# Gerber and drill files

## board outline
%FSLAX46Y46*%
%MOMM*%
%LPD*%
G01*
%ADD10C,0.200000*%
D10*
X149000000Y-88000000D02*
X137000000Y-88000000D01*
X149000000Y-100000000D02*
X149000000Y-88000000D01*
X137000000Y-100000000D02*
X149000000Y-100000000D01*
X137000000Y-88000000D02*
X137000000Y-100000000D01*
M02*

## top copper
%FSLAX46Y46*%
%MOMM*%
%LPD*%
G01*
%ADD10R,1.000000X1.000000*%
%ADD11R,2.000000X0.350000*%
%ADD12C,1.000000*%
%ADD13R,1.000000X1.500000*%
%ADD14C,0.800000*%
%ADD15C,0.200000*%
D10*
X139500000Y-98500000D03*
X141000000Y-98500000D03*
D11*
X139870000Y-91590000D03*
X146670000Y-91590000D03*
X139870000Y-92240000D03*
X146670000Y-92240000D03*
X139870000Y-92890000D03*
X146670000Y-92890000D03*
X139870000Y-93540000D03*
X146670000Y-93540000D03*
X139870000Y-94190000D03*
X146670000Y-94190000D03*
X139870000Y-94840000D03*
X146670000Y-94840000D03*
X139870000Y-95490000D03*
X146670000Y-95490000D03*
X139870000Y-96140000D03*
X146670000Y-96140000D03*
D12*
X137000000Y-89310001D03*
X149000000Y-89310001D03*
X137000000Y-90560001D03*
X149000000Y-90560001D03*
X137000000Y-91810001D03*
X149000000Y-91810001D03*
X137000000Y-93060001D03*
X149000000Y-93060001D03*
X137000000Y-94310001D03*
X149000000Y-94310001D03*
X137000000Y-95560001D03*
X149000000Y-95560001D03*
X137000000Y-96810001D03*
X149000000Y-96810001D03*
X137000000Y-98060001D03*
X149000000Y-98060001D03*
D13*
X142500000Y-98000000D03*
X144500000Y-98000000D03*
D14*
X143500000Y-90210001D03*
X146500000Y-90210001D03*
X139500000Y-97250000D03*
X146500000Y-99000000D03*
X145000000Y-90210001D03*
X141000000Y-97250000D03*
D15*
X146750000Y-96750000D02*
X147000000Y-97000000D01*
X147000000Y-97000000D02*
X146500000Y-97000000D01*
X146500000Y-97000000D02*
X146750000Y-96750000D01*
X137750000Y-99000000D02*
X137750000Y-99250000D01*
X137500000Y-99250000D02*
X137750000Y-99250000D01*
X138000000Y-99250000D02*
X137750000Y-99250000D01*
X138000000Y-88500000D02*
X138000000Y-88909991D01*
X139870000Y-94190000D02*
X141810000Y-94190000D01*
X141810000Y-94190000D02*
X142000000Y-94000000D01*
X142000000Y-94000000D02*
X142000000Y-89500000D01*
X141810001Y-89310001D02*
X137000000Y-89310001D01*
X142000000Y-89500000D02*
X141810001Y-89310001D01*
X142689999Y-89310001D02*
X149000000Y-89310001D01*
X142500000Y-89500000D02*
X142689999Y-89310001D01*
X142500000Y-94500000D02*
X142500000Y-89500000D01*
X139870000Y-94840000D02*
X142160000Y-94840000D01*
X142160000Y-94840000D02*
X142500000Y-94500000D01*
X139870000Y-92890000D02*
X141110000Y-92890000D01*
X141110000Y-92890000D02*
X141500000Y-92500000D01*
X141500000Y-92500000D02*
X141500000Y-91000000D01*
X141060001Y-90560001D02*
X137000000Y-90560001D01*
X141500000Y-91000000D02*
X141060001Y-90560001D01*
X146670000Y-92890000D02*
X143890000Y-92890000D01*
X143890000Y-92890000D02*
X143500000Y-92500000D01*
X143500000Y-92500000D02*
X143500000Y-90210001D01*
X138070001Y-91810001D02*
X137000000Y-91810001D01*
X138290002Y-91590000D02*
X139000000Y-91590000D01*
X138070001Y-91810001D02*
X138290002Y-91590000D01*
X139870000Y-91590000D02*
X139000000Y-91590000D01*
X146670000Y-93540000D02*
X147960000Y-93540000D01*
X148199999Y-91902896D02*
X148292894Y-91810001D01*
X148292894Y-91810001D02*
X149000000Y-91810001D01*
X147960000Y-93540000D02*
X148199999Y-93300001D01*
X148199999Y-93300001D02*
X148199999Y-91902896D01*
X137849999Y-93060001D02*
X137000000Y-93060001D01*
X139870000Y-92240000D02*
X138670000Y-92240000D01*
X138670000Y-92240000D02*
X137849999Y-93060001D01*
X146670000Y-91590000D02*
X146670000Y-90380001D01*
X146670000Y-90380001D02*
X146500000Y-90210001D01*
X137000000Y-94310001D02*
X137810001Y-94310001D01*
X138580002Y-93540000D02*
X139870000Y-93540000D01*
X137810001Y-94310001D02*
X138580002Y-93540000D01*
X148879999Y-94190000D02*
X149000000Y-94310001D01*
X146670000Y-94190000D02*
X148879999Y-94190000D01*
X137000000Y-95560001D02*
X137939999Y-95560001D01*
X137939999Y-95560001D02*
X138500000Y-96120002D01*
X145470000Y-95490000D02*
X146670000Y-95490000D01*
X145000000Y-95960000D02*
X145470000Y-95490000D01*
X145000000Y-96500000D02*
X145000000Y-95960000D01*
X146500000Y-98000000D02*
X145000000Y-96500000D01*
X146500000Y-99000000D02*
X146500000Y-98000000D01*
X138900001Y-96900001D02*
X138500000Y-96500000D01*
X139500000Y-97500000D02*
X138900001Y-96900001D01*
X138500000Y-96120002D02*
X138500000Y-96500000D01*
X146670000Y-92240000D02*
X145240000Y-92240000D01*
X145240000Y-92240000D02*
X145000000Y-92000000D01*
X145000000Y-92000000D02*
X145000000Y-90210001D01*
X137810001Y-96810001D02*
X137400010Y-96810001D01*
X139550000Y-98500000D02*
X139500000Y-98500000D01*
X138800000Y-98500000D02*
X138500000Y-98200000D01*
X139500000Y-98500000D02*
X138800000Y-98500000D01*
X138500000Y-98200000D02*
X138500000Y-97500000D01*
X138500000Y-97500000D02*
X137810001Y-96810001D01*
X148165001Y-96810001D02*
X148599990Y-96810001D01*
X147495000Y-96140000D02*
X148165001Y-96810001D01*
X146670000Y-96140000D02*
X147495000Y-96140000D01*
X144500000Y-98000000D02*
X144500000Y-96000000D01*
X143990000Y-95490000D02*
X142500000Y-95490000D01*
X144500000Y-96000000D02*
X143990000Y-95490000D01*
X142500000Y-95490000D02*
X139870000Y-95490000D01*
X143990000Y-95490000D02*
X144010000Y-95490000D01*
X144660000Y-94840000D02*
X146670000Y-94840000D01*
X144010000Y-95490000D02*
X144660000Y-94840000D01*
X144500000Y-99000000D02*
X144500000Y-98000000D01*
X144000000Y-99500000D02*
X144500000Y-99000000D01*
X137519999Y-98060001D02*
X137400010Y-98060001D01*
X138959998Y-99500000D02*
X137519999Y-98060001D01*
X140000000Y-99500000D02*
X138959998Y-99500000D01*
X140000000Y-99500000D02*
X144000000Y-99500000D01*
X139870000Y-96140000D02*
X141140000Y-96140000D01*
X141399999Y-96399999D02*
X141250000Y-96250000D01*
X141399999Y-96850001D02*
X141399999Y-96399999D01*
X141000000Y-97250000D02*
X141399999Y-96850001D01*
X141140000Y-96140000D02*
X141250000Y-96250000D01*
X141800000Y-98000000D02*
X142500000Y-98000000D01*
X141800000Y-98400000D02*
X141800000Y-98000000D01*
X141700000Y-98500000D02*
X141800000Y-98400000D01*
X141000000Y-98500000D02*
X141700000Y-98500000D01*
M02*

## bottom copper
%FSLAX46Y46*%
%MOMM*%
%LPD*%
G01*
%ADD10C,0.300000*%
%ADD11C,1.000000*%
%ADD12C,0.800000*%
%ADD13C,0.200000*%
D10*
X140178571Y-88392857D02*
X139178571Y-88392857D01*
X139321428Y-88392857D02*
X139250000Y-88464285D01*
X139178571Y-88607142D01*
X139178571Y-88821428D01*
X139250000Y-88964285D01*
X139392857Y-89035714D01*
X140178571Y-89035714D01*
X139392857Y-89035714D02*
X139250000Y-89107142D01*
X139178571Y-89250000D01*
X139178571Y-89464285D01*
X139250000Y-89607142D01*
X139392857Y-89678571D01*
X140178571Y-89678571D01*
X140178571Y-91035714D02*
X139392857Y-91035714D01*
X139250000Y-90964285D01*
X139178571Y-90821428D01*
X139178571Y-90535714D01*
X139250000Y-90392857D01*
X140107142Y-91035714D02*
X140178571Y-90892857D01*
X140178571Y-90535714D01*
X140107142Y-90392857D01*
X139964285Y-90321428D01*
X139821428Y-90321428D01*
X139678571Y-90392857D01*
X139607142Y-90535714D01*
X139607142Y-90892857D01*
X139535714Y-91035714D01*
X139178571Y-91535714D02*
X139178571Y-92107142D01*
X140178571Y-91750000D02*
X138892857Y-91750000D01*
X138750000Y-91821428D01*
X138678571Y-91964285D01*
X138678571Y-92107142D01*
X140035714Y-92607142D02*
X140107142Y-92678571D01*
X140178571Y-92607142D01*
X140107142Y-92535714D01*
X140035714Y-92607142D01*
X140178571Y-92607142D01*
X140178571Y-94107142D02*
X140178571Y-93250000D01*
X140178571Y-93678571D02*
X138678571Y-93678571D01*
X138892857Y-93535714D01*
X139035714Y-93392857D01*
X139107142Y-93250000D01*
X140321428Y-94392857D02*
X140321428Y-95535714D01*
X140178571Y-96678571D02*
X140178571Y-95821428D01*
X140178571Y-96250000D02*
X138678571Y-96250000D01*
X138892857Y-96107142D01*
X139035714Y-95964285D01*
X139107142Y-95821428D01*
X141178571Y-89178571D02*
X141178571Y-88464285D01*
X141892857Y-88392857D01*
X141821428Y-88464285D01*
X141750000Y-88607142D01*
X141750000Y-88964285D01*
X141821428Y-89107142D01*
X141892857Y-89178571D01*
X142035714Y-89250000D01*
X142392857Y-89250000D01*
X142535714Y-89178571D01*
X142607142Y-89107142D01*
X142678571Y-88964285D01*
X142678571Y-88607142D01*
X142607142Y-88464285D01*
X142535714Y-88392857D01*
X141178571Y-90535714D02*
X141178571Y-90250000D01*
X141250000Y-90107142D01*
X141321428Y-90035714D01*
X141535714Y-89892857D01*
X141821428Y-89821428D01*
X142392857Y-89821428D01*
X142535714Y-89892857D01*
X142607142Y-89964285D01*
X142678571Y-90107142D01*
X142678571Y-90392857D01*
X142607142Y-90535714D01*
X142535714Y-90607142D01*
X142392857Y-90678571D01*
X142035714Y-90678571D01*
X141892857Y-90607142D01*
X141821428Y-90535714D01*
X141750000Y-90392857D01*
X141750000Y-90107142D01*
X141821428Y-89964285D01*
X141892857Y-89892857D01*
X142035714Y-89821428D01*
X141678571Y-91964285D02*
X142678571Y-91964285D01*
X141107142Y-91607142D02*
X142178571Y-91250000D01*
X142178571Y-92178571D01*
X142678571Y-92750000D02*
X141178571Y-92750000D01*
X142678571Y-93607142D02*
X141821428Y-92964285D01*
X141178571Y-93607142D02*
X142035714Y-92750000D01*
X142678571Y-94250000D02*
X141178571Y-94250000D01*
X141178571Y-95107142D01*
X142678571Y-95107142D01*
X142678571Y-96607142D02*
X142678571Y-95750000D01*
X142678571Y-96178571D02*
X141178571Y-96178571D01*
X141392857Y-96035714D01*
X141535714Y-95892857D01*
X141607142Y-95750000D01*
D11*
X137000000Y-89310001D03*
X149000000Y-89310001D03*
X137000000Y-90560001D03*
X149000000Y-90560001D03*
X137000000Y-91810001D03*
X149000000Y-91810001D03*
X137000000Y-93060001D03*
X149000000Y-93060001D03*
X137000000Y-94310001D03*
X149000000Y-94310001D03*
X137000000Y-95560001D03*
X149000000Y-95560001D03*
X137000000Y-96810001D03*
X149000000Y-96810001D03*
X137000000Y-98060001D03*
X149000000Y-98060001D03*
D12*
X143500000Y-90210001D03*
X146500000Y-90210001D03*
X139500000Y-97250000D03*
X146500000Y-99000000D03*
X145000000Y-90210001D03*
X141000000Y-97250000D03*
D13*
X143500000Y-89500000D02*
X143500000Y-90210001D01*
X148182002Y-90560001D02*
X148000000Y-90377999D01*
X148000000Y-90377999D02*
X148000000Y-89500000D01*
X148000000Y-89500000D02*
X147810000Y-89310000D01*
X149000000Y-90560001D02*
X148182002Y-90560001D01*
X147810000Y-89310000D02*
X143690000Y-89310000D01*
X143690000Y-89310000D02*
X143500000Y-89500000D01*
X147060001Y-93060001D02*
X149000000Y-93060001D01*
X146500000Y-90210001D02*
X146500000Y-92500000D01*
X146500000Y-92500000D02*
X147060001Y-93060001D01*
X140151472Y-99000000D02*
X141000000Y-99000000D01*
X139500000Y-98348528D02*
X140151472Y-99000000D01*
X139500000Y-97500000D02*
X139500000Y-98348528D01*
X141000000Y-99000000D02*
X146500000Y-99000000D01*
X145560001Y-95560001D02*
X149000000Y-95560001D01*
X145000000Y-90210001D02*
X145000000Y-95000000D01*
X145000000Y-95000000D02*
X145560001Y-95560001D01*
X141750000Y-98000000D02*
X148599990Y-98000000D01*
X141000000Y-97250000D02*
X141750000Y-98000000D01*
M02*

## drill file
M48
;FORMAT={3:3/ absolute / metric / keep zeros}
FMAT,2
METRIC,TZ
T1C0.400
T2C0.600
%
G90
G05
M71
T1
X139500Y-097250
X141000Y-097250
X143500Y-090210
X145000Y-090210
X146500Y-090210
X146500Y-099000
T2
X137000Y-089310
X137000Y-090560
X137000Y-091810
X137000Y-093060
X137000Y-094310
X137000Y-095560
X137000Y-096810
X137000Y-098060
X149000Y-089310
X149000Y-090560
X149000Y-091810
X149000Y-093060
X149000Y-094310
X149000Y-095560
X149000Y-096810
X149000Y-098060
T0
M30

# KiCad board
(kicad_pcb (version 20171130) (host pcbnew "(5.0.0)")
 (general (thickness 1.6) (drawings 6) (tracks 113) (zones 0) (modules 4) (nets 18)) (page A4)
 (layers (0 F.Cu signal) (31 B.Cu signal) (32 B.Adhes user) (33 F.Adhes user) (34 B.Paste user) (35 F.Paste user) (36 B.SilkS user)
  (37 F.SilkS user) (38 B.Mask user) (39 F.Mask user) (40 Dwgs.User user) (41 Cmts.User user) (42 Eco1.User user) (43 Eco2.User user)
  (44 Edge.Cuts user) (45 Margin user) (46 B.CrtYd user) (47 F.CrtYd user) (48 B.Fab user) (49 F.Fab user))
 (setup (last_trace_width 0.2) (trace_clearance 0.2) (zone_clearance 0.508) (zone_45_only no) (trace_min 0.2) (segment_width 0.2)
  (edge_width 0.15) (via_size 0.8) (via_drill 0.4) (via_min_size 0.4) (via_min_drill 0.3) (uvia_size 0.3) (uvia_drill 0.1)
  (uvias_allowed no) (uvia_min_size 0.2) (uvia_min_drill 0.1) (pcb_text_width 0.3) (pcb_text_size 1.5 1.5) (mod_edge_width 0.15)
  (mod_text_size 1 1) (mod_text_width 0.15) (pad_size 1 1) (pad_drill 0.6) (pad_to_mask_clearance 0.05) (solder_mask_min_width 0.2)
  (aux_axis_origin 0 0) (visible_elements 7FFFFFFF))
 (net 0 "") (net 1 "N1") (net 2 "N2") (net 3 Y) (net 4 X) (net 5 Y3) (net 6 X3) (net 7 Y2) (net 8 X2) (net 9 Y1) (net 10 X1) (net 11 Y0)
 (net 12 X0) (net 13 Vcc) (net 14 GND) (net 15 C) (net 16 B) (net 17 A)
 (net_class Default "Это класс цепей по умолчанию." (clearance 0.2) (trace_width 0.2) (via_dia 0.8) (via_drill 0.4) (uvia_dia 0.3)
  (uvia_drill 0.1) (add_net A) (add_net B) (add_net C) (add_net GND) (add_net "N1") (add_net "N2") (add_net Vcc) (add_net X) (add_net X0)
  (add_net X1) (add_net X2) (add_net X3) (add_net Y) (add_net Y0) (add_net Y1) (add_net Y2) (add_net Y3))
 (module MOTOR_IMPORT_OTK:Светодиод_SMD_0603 (layer F.Cu) (at 141 98.5 180)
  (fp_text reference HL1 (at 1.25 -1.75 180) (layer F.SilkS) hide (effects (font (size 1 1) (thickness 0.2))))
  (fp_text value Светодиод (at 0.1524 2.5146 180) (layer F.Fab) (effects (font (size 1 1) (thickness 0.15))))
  (pad 2 smd rect (at 1.5 0 180) (size 1 1) (layers F.Cu F.Paste F.Mask) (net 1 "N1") (clearance 0.2))
  (pad 1 smd rect (at 0 0 180) (size 1 1) (layers F.Cu F.Paste F.Mask) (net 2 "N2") (clearance 0.2)))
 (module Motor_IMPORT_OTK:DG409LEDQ (layer F.Cu) (at 145.5 89.5 180)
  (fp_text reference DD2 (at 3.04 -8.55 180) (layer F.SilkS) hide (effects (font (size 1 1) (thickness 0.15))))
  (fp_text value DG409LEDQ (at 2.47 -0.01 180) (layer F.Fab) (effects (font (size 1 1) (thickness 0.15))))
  (pad 9 smd rect (at 5.63 -2.09 180) (size 2 0.35) (layers F.Cu F.Paste F.Mask) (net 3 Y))
  (pad 8 smd rect (at -1.17 -2.09 180) (size 2 0.35) (layers F.Cu F.Paste F.Mask) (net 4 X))
  (pad 10 smd rect (at 5.63 -2.74 180) (size 2 0.35) (layers F.Cu F.Paste F.Mask) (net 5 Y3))
  (pad 7 smd rect (at -1.17 -2.74 180) (size 2 0.35) (layers F.Cu F.Paste F.Mask) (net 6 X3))
  (pad 11 smd rect (at 5.63 -3.39 180) (size 2 0.35) (layers F.Cu F.Paste F.Mask) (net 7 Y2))
  (pad 6 smd rect (at -1.17 -3.39 180) (size 2 0.35) (layers F.Cu F.Paste F.Mask) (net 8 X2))
  (pad 12 smd rect (at 5.63 -4.04 180) (size 2 0.35) (layers F.Cu F.Paste F.Mask) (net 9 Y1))
  (pad 5 smd rect (at -1.17 -4.04 180) (size 2 0.35) (layers F.Cu F.Paste F.Mask) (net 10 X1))
  (pad 13 smd rect (at 5.63 -4.69 180) (size 2 0.35) (layers F.Cu F.Paste F.Mask) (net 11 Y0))
  (pad 4 smd rect (at -1.17 -4.69 180) (size 2 0.35) (layers F.Cu F.Paste F.Mask) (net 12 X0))
  (pad 14 smd rect (at 5.63 -5.34 180) (size 2 0.35) (layers F.Cu F.Paste F.Mask) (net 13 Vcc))
  (pad 3 smd rect (at -1.17 -5.34 180) (size 2 0.35) (layers F.Cu F.Paste F.Mask) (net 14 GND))
  (pad 15 smd rect (at 5.63 -5.99 180) (size 2 0.35) (layers F.Cu F.Paste F.Mask) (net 14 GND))
  (pad 2 smd rect (at -1.17 -5.99 180) (size 2 0.35) (layers F.Cu F.Paste F.Mask) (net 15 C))
  (pad 16 smd rect (at 5.63 -6.64 180) (size 2 0.35) (layers F.Cu F.Paste F.Mask) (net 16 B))
  (pad 1 smd rect (at -1.17 -6.64 180) (size 2 0.35) (layers F.Cu F.Paste F.Mask) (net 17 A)))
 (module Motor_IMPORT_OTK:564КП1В (layer F.Cu) (at 137 106.650001)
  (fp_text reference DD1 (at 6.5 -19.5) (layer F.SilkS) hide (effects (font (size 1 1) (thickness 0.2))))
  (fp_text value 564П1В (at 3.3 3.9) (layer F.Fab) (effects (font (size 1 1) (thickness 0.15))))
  (pad 1 thru_hole circle (at 0 -17.34) (size 1 1) (drill 0.6) (layers *.Cu *.Mask) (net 11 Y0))
  (pad 16 thru_hole circle (at 12 -17.34) (size 1 1) (drill 0.6) (layers *.Cu *.Mask) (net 13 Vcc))
  (pad 2 thru_hole circle (at 0 -16.09) (size 1 1) (drill 0.6) (layers *.Cu *.Mask) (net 7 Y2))
  (pad 15 thru_hole circle (at 12 -16.09) (size 1 1) (drill 0.6) (layers *.Cu *.Mask) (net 8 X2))
  (pad 3 thru_hole circle (at 0 -14.84) (size 1 1) (drill 0.6) (layers *.Cu *.Mask) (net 3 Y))
  (pad 14 thru_hole circle (at 12 -14.84) (size 1 1) (drill 0.6) (layers *.Cu *.Mask) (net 10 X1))
  (pad 4 thru_hole circle (at 0 -13.59) (size 1 1) (drill 0.6) (layers *.Cu *.Mask) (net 5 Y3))
  (pad 13 thru_hole circle (at 12 -13.59) (size 1 1) (drill 0.6) (layers *.Cu *.Mask) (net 4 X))
  (pad 5 thru_hole circle (at 0 -12.34) (size 1 1) (drill 0.6) (layers *.Cu *.Mask) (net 9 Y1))
  (pad 12 thru_hole circle (at 12 -12.34) (size 1 1) (drill 0.6) (layers *.Cu *.Mask) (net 12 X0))
  (pad 6 thru_hole circle (at 0 -11.09) (size 1 1) (drill 0.6) (layers *.Cu *.Mask) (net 15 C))
  (pad 11 thru_hole circle (at 12 -11.09) (size 1 1) (drill 0.6) (layers *.Cu *.Mask) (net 6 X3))
  (pad 7 thru_hole circle (at 0 -9.84) (size 1 1) (drill 0.6) (layers *.Cu *.Mask) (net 1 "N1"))
  (pad 10 thru_hole circle (at 12 -9.84) (size 1 1) (drill 0.6) (layers *.Cu *.Mask) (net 17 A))
  (pad 8 thru_hole circle (at 0 -8.59) (size 1 1) (drill 0.6) (layers *.Cu *.Mask) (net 14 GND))
  (pad 9 thru_hole circle (at 12 -8.59) (size 1 1) (drill 0.6) (layers *.Cu *.Mask) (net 16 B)))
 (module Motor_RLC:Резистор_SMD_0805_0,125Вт (layer F.Cu) (at 144.5 98 180)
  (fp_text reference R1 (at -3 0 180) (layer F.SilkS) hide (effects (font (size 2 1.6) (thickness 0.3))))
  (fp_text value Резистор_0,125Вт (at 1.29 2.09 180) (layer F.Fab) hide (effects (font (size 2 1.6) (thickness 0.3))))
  (pad 2 smd rect (at 2 0 180) (size 1 1.5) (layers F.Cu F.Paste F.Mask) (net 2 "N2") (clearance 0.2))
  (pad 1 smd rect (at 0 0 180) (size 1 1.5) (layers F.Cu F.Paste F.Mask) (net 14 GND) (clearance 0.2)))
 (gr_line (start 149 88) (end 137 88) (layer Edge.Cuts) (width 0.2))
 (gr_line (start 149 100) (end 149 88) (layer Edge.Cuts) (width 0.2))
 (gr_line (start 137 100) (end 149 100) (layer Edge.Cuts) (width 0.2))
 (gr_line (start 137 88) (end 137 100) (layer Edge.Cuts) (width 0.2))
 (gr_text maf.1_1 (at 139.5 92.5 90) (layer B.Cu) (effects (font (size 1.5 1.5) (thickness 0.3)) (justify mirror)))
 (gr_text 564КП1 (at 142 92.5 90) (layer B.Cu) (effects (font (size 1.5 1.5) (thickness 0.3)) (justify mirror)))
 (segment (start 146.75 96.75) (end 147 97) (width 0.2) (layer F.Cu) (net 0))
 (segment (start 147 97) (end 146.5 97) (width 0.2) (layer F.Cu) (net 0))
 (segment (start 146.5 97) (end 146.75 96.75) (width 0.2) (layer F.Cu) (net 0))
 (segment (start 137.75 99) (end 137.75 99.25) (width 0.2) (layer F.Cu) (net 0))
 (segment (start 137.5 99.25) (end 137.75 99.25) (width 0.2) (layer F.Cu) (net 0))
 (segment (start 138 99.25) (end 137.75 99.25) (width 0.2) (layer F.Cu) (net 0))
 (segment (start 138 88.5) (end 138 88.909991) (width 0.2) (layer F.Cu) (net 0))
 (segment (start 139.87 94.19) (end 141.81 94.19) (width 0.2) (layer F.Cu) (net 11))
 (segment (start 141.81 94.19) (end 142 94) (width 0.2) (layer F.Cu) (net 11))
 (segment (start 142 94) (end 142 89.5) (width 0.2) (layer F.Cu) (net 11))
 (segment (start 141.810001 89.310001) (end 137 89.310001) (width 0.2) (layer F.Cu) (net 11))
 (segment (start 142 89.5) (end 141.810001 89.310001) (width 0.2) (layer F.Cu) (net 11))
 (segment (start 142.689999 89.310001) (end 149 89.310001) (width 0.2) (layer F.Cu) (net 13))
 (segment (start 142.5 89.5) (end 142.689999 89.310001) (width 0.2) (layer F.Cu) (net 13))
 (segment (start 142.5 94.5) (end 142.5 89.5) (width 0.2) (layer F.Cu) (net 13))
 (segment (start 139.87 94.84) (end 142.16 94.84) (width 0.2) (layer F.Cu) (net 13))
 (segment (start 142.16 94.84) (end 142.5 94.5) (width 0.2) (layer F.Cu) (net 13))
 (segment (start 139.87 92.89) (end 141.11 92.89) (width 0.2) (layer F.Cu) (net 7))
 (segment (start 141.11 92.89) (end 141.5 92.5) (width 0.2) (layer F.Cu) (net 7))
 (segment (start 141.5 92.5) (end 141.5 91) (width 0.2) (layer F.Cu) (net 7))
 (segment (start 141.060001 90.560001) (end 137 90.560001) (width 0.2) (layer F.Cu) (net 7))
 (segment (start 141.5 91) (end 141.060001 90.560001) (width 0.2) (layer F.Cu) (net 7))
 (segment (start 146.67 92.89) (end 143.89 92.89) (width 0.2) (layer F.Cu) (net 8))
 (via (at 143.5 90.210001) (size 0.8) (drill 0.4) (layers F.Cu B.Cu) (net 8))
 (segment (start 143.89 92.89) (end 143.5 92.5) (width 0.2) (layer F.Cu) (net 8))
 (segment (start 143.5 92.5) (end 143.5 90.210001) (width 0.2) (layer F.Cu) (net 8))
 (segment (start 143.5 89.5) (end 143.5 90.210001) (width 0.2) (layer B.Cu) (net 8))
 (segment (start 148.182002 90.560001) (end 148 90.377999) (width 0.2) (layer B.Cu) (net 8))
 (segment (start 148 90.377999) (end 148 89.5) (width 0.2) (layer B.Cu) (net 8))
 (segment (start 148 89.5) (end 147.81 89.31) (width 0.2) (layer B.Cu) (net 8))
 (segment (start 149 90.560001) (end 148.182002 90.560001) (width 0.2) (layer B.Cu) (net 8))
 (segment (start 147.81 89.31) (end 143.69 89.31) (width 0.2) (layer B.Cu) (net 8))
 (segment (start 143.69 89.31) (end 143.5 89.5) (width 0.2) (layer B.Cu) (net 8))
 (segment (start 138.070001 91.810001) (end 137 91.810001) (width 0.2) (layer F.Cu) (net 3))
 (segment (start 138.290002 91.59) (end 139 91.59) (width 0.2) (layer F.Cu) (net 3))
 (segment (start 138.070001 91.810001) (end 138.290002 91.59) (width 0.2) (layer F.Cu) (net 3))
 (segment (start 139.87 91.59) (end 139 91.59) (width 0.2) (layer F.Cu) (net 3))
 (segment (start 146.67 93.54) (end 147.96 93.54) (width 0.2) (layer F.Cu) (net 10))
 (segment (start 148.199999 91.902896) (end 148.292894 91.810001) (width 0.2) (layer F.Cu) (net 10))
 (segment (start 148.292894 91.810001) (end 149 91.810001) (width 0.2) (layer F.Cu) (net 10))
 (segment (start 147.96 93.54) (end 148.199999 93.300001) (width 0.2) (layer F.Cu) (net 10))
 (segment (start 148.199999 93.300001) (end 148.199999 91.902896) (width 0.2) (layer F.Cu) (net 10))
 (segment (start 137.849999 93.060001) (end 137 93.060001) (width 0.2) (layer F.Cu) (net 5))
 (segment (start 139.87 92.24) (end 138.67 92.24) (width 0.2) (layer F.Cu) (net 5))
 (segment (start 138.67 92.24) (end 137.849999 93.060001) (width 0.2) (layer F.Cu) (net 5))
 (via (at 146.5 90.210001) (size 0.8) (drill 0.4) (layers F.Cu B.Cu) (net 4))
 (segment (start 146.67 91.59) (end 146.67 90.380001) (width 0.2) (layer F.Cu) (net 4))
 (segment (start 146.67 90.380001) (end 146.5 90.210001) (width 0.2) (layer F.Cu) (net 4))
 (segment (start 147.060001 93.060001) (end 149 93.060001) (width 0.2) (layer B.Cu) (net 4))
 (segment (start 146.5 90.210001) (end 146.5 92.5) (width 0.2) (layer B.Cu) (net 4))
 (segment (start 146.5 92.5) (end 147.060001 93.060001) (width 0.2) (layer B.Cu) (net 4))
 (segment (start 137 94.310001) (end 137.810001 94.310001) (width 0.2) (layer F.Cu) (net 9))
 (segment (start 138.580002 93.54) (end 139.87 93.54) (width 0.2) (layer F.Cu) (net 9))
 (segment (start 137.810001 94.310001) (end 138.580002 93.54) (width 0.2) (layer F.Cu) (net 9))
 (segment (start 148.879999 94.19) (end 149 94.310001) (width 0.2) (layer F.Cu) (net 12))
 (segment (start 146.67 94.19) (end 148.879999 94.19) (width 0.2) (layer F.Cu) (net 12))
 (segment (start 137 95.560001) (end 137.939999 95.560001) (width 0.2) (layer F.Cu) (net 15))
 (via (at 139.5 97.25) (size 0.8) (drill 0.4) (layers F.Cu B.Cu) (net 15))
 (segment (start 137.939999 95.560001) (end 138.5 96.120002) (width 0.2) (layer F.Cu) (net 15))
 (via (at 146.5 99) (size 0.8) (drill 0.4) (layers F.Cu B.Cu) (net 15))
 (segment (start 145.47 95.49) (end 146.67 95.49) (width 0.2) (layer F.Cu) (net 15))
 (segment (start 145 95.96) (end 145.47 95.49) (width 0.2) (layer F.Cu) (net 15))
 (segment (start 145 96.5) (end 145 95.96) (width 0.2) (layer F.Cu) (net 15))
 (segment (start 146.5 98) (end 145 96.5) (width 0.2) (layer F.Cu) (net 15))
 (segment (start 146.5 99) (end 146.5 98) (width 0.2) (layer F.Cu) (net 15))
 (segment (start 138.900001 96.900001) (end 138.5 96.5) (width 0.2) (layer F.Cu) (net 15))
 (segment (start 139.5 97.5) (end 138.900001 96.900001) (width 0.2) (layer F.Cu) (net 15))
 (segment (start 138.5 96.120002) (end 138.5 96.5) (width 0.2) (layer F.Cu) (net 15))
 (segment (start 140.151472 99) (end 141 99) (width 0.2) (layer B.Cu) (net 15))
 (segment (start 139.5 98.348528) (end 140.151472 99) (width 0.2) (layer B.Cu) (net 15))
 (segment (start 139.5 97.5) (end 139.5 98.348528) (width 0.2) (layer B.Cu) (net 15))
 (segment (start 141 99) (end 146.5 99) (width 0.2) (layer B.Cu) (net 15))
 (segment (start 146.67 92.24) (end 145.24 92.24) (width 0.2) (layer F.Cu) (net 6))
 (via (at 145 90.210001) (size 0.8) (drill 0.4) (layers F.Cu B.Cu) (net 6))
 (segment (start 145.24 92.24) (end 145 92) (width 0.2) (layer F.Cu) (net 6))
 (segment (start 145 92) (end 145 90.210001) (width 0.2) (layer F.Cu) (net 6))
 (segment (start 145.560001 95.560001) (end 149 95.560001) (width 0.2) (layer B.Cu) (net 6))
 (segment (start 145 90.210001) (end 145 95) (width 0.2) (layer B.Cu) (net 6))
 (segment (start 145 95) (end 145.560001 95.560001) (width 0.2) (layer B.Cu) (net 6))
 (segment (start 137.810001 96.810001) (end 137.40001 96.810001) (width 0.2) (layer F.Cu) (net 1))
 (segment (start 139.55 98.5) (end 139.5 98.5) (width 0.2) (layer F.Cu) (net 1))
 (segment (start 138.8 98.5) (end 138.5 98.2) (width 0.2) (layer F.Cu) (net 1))
 (segment (start 139.5 98.5) (end 138.8 98.5) (width 0.2) (layer F.Cu) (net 1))
 (segment (start 138.5 98.2) (end 138.5 97.5) (width 0.2) (layer F.Cu) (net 1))
 (segment (start 138.5 97.5) (end 137.810001 96.810001) (width 0.2) (layer F.Cu) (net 1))
 (segment (start 148.165001 96.810001) (end 148.59999 96.810001) (width 0.2) (layer F.Cu) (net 17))
 (segment (start 147.495 96.14) (end 148.165001 96.810001) (width 0.2) (layer F.Cu) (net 17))
 (segment (start 146.67 96.14) (end 147.495 96.14) (width 0.2) (layer F.Cu) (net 17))
 (segment (start 144.5 98) (end 144.5 96) (width 0.2) (layer F.Cu) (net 14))
 (segment (start 143.99 95.49) (end 142.5 95.49) (width 0.2) (layer F.Cu) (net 14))
 (segment (start 144.5 96) (end 143.99 95.49) (width 0.2) (layer F.Cu) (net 14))
 (segment (start 142.5 95.49) (end 139.87 95.49) (width 0.2) (layer F.Cu) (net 14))
 (segment (start 143.99 95.49) (end 144.01 95.49) (width 0.2) (layer F.Cu) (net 14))
 (segment (start 144.66 94.84) (end 146.67 94.84) (width 0.2) (layer F.Cu) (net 14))
 (segment (start 144.01 95.49) (end 144.66 94.84) (width 0.2) (layer F.Cu) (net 14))
 (segment (start 144.5 99) (end 144.5 98) (width 0.2) (layer F.Cu) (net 14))
 (segment (start 144 99.5) (end 144.5 99) (width 0.2) (layer F.Cu) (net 14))
 (segment (start 137.519999 98.060001) (end 137.40001 98.060001) (width 0.2) (layer F.Cu) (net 14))
 (segment (start 138.959998 99.5) (end 137.519999 98.060001) (width 0.2) (layer F.Cu) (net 14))
 (segment (start 140 99.5) (end 138.959998 99.5) (width 0.2) (layer F.Cu) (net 14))
 (segment (start 140 99.5) (end 144 99.5) (width 0.2) (layer F.Cu) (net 14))
 (segment (start 139.87 96.14) (end 141.14 96.14) (width 0.2) (layer F.Cu) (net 16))
 (segment (start 141.399999 96.399999) (end 141.25 96.25) (width 0.2) (layer F.Cu) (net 16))
 (segment (start 141.399999 96.850001) (end 141.399999 96.399999) (width 0.2) (layer F.Cu) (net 16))
 (segment (start 141 97.25) (end 141.399999 96.850001) (width 0.2) (layer F.Cu) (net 16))
 (segment (start 141.14 96.14) (end 141.25 96.25) (width 0.2) (layer F.Cu) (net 16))
 (via (at 141 97.25) (size 0.8) (drill 0.4) (layers F.Cu B.Cu) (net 16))
 (segment (start 141.75 98) (end 148.59999 98) (width 0.2) (layer B.Cu) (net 16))
 (segment (start 141 97.25) (end 141.75 98) (width 0.2) (layer B.Cu) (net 16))
 (segment (start 141.8 98) (end 142.5 98) (width 0.2) (layer F.Cu) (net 2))
 (segment (start 141.8 98.4) (end 141.8 98) (width 0.2) (layer F.Cu) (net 2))
 (segment (start 141.7 98.5) (end 141.8 98.4) (width 0.2) (layer F.Cu) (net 2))
 (segment (start 141 98.5) (end 141.7 98.5) (width 0.2) (layer F.Cu) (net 2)))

